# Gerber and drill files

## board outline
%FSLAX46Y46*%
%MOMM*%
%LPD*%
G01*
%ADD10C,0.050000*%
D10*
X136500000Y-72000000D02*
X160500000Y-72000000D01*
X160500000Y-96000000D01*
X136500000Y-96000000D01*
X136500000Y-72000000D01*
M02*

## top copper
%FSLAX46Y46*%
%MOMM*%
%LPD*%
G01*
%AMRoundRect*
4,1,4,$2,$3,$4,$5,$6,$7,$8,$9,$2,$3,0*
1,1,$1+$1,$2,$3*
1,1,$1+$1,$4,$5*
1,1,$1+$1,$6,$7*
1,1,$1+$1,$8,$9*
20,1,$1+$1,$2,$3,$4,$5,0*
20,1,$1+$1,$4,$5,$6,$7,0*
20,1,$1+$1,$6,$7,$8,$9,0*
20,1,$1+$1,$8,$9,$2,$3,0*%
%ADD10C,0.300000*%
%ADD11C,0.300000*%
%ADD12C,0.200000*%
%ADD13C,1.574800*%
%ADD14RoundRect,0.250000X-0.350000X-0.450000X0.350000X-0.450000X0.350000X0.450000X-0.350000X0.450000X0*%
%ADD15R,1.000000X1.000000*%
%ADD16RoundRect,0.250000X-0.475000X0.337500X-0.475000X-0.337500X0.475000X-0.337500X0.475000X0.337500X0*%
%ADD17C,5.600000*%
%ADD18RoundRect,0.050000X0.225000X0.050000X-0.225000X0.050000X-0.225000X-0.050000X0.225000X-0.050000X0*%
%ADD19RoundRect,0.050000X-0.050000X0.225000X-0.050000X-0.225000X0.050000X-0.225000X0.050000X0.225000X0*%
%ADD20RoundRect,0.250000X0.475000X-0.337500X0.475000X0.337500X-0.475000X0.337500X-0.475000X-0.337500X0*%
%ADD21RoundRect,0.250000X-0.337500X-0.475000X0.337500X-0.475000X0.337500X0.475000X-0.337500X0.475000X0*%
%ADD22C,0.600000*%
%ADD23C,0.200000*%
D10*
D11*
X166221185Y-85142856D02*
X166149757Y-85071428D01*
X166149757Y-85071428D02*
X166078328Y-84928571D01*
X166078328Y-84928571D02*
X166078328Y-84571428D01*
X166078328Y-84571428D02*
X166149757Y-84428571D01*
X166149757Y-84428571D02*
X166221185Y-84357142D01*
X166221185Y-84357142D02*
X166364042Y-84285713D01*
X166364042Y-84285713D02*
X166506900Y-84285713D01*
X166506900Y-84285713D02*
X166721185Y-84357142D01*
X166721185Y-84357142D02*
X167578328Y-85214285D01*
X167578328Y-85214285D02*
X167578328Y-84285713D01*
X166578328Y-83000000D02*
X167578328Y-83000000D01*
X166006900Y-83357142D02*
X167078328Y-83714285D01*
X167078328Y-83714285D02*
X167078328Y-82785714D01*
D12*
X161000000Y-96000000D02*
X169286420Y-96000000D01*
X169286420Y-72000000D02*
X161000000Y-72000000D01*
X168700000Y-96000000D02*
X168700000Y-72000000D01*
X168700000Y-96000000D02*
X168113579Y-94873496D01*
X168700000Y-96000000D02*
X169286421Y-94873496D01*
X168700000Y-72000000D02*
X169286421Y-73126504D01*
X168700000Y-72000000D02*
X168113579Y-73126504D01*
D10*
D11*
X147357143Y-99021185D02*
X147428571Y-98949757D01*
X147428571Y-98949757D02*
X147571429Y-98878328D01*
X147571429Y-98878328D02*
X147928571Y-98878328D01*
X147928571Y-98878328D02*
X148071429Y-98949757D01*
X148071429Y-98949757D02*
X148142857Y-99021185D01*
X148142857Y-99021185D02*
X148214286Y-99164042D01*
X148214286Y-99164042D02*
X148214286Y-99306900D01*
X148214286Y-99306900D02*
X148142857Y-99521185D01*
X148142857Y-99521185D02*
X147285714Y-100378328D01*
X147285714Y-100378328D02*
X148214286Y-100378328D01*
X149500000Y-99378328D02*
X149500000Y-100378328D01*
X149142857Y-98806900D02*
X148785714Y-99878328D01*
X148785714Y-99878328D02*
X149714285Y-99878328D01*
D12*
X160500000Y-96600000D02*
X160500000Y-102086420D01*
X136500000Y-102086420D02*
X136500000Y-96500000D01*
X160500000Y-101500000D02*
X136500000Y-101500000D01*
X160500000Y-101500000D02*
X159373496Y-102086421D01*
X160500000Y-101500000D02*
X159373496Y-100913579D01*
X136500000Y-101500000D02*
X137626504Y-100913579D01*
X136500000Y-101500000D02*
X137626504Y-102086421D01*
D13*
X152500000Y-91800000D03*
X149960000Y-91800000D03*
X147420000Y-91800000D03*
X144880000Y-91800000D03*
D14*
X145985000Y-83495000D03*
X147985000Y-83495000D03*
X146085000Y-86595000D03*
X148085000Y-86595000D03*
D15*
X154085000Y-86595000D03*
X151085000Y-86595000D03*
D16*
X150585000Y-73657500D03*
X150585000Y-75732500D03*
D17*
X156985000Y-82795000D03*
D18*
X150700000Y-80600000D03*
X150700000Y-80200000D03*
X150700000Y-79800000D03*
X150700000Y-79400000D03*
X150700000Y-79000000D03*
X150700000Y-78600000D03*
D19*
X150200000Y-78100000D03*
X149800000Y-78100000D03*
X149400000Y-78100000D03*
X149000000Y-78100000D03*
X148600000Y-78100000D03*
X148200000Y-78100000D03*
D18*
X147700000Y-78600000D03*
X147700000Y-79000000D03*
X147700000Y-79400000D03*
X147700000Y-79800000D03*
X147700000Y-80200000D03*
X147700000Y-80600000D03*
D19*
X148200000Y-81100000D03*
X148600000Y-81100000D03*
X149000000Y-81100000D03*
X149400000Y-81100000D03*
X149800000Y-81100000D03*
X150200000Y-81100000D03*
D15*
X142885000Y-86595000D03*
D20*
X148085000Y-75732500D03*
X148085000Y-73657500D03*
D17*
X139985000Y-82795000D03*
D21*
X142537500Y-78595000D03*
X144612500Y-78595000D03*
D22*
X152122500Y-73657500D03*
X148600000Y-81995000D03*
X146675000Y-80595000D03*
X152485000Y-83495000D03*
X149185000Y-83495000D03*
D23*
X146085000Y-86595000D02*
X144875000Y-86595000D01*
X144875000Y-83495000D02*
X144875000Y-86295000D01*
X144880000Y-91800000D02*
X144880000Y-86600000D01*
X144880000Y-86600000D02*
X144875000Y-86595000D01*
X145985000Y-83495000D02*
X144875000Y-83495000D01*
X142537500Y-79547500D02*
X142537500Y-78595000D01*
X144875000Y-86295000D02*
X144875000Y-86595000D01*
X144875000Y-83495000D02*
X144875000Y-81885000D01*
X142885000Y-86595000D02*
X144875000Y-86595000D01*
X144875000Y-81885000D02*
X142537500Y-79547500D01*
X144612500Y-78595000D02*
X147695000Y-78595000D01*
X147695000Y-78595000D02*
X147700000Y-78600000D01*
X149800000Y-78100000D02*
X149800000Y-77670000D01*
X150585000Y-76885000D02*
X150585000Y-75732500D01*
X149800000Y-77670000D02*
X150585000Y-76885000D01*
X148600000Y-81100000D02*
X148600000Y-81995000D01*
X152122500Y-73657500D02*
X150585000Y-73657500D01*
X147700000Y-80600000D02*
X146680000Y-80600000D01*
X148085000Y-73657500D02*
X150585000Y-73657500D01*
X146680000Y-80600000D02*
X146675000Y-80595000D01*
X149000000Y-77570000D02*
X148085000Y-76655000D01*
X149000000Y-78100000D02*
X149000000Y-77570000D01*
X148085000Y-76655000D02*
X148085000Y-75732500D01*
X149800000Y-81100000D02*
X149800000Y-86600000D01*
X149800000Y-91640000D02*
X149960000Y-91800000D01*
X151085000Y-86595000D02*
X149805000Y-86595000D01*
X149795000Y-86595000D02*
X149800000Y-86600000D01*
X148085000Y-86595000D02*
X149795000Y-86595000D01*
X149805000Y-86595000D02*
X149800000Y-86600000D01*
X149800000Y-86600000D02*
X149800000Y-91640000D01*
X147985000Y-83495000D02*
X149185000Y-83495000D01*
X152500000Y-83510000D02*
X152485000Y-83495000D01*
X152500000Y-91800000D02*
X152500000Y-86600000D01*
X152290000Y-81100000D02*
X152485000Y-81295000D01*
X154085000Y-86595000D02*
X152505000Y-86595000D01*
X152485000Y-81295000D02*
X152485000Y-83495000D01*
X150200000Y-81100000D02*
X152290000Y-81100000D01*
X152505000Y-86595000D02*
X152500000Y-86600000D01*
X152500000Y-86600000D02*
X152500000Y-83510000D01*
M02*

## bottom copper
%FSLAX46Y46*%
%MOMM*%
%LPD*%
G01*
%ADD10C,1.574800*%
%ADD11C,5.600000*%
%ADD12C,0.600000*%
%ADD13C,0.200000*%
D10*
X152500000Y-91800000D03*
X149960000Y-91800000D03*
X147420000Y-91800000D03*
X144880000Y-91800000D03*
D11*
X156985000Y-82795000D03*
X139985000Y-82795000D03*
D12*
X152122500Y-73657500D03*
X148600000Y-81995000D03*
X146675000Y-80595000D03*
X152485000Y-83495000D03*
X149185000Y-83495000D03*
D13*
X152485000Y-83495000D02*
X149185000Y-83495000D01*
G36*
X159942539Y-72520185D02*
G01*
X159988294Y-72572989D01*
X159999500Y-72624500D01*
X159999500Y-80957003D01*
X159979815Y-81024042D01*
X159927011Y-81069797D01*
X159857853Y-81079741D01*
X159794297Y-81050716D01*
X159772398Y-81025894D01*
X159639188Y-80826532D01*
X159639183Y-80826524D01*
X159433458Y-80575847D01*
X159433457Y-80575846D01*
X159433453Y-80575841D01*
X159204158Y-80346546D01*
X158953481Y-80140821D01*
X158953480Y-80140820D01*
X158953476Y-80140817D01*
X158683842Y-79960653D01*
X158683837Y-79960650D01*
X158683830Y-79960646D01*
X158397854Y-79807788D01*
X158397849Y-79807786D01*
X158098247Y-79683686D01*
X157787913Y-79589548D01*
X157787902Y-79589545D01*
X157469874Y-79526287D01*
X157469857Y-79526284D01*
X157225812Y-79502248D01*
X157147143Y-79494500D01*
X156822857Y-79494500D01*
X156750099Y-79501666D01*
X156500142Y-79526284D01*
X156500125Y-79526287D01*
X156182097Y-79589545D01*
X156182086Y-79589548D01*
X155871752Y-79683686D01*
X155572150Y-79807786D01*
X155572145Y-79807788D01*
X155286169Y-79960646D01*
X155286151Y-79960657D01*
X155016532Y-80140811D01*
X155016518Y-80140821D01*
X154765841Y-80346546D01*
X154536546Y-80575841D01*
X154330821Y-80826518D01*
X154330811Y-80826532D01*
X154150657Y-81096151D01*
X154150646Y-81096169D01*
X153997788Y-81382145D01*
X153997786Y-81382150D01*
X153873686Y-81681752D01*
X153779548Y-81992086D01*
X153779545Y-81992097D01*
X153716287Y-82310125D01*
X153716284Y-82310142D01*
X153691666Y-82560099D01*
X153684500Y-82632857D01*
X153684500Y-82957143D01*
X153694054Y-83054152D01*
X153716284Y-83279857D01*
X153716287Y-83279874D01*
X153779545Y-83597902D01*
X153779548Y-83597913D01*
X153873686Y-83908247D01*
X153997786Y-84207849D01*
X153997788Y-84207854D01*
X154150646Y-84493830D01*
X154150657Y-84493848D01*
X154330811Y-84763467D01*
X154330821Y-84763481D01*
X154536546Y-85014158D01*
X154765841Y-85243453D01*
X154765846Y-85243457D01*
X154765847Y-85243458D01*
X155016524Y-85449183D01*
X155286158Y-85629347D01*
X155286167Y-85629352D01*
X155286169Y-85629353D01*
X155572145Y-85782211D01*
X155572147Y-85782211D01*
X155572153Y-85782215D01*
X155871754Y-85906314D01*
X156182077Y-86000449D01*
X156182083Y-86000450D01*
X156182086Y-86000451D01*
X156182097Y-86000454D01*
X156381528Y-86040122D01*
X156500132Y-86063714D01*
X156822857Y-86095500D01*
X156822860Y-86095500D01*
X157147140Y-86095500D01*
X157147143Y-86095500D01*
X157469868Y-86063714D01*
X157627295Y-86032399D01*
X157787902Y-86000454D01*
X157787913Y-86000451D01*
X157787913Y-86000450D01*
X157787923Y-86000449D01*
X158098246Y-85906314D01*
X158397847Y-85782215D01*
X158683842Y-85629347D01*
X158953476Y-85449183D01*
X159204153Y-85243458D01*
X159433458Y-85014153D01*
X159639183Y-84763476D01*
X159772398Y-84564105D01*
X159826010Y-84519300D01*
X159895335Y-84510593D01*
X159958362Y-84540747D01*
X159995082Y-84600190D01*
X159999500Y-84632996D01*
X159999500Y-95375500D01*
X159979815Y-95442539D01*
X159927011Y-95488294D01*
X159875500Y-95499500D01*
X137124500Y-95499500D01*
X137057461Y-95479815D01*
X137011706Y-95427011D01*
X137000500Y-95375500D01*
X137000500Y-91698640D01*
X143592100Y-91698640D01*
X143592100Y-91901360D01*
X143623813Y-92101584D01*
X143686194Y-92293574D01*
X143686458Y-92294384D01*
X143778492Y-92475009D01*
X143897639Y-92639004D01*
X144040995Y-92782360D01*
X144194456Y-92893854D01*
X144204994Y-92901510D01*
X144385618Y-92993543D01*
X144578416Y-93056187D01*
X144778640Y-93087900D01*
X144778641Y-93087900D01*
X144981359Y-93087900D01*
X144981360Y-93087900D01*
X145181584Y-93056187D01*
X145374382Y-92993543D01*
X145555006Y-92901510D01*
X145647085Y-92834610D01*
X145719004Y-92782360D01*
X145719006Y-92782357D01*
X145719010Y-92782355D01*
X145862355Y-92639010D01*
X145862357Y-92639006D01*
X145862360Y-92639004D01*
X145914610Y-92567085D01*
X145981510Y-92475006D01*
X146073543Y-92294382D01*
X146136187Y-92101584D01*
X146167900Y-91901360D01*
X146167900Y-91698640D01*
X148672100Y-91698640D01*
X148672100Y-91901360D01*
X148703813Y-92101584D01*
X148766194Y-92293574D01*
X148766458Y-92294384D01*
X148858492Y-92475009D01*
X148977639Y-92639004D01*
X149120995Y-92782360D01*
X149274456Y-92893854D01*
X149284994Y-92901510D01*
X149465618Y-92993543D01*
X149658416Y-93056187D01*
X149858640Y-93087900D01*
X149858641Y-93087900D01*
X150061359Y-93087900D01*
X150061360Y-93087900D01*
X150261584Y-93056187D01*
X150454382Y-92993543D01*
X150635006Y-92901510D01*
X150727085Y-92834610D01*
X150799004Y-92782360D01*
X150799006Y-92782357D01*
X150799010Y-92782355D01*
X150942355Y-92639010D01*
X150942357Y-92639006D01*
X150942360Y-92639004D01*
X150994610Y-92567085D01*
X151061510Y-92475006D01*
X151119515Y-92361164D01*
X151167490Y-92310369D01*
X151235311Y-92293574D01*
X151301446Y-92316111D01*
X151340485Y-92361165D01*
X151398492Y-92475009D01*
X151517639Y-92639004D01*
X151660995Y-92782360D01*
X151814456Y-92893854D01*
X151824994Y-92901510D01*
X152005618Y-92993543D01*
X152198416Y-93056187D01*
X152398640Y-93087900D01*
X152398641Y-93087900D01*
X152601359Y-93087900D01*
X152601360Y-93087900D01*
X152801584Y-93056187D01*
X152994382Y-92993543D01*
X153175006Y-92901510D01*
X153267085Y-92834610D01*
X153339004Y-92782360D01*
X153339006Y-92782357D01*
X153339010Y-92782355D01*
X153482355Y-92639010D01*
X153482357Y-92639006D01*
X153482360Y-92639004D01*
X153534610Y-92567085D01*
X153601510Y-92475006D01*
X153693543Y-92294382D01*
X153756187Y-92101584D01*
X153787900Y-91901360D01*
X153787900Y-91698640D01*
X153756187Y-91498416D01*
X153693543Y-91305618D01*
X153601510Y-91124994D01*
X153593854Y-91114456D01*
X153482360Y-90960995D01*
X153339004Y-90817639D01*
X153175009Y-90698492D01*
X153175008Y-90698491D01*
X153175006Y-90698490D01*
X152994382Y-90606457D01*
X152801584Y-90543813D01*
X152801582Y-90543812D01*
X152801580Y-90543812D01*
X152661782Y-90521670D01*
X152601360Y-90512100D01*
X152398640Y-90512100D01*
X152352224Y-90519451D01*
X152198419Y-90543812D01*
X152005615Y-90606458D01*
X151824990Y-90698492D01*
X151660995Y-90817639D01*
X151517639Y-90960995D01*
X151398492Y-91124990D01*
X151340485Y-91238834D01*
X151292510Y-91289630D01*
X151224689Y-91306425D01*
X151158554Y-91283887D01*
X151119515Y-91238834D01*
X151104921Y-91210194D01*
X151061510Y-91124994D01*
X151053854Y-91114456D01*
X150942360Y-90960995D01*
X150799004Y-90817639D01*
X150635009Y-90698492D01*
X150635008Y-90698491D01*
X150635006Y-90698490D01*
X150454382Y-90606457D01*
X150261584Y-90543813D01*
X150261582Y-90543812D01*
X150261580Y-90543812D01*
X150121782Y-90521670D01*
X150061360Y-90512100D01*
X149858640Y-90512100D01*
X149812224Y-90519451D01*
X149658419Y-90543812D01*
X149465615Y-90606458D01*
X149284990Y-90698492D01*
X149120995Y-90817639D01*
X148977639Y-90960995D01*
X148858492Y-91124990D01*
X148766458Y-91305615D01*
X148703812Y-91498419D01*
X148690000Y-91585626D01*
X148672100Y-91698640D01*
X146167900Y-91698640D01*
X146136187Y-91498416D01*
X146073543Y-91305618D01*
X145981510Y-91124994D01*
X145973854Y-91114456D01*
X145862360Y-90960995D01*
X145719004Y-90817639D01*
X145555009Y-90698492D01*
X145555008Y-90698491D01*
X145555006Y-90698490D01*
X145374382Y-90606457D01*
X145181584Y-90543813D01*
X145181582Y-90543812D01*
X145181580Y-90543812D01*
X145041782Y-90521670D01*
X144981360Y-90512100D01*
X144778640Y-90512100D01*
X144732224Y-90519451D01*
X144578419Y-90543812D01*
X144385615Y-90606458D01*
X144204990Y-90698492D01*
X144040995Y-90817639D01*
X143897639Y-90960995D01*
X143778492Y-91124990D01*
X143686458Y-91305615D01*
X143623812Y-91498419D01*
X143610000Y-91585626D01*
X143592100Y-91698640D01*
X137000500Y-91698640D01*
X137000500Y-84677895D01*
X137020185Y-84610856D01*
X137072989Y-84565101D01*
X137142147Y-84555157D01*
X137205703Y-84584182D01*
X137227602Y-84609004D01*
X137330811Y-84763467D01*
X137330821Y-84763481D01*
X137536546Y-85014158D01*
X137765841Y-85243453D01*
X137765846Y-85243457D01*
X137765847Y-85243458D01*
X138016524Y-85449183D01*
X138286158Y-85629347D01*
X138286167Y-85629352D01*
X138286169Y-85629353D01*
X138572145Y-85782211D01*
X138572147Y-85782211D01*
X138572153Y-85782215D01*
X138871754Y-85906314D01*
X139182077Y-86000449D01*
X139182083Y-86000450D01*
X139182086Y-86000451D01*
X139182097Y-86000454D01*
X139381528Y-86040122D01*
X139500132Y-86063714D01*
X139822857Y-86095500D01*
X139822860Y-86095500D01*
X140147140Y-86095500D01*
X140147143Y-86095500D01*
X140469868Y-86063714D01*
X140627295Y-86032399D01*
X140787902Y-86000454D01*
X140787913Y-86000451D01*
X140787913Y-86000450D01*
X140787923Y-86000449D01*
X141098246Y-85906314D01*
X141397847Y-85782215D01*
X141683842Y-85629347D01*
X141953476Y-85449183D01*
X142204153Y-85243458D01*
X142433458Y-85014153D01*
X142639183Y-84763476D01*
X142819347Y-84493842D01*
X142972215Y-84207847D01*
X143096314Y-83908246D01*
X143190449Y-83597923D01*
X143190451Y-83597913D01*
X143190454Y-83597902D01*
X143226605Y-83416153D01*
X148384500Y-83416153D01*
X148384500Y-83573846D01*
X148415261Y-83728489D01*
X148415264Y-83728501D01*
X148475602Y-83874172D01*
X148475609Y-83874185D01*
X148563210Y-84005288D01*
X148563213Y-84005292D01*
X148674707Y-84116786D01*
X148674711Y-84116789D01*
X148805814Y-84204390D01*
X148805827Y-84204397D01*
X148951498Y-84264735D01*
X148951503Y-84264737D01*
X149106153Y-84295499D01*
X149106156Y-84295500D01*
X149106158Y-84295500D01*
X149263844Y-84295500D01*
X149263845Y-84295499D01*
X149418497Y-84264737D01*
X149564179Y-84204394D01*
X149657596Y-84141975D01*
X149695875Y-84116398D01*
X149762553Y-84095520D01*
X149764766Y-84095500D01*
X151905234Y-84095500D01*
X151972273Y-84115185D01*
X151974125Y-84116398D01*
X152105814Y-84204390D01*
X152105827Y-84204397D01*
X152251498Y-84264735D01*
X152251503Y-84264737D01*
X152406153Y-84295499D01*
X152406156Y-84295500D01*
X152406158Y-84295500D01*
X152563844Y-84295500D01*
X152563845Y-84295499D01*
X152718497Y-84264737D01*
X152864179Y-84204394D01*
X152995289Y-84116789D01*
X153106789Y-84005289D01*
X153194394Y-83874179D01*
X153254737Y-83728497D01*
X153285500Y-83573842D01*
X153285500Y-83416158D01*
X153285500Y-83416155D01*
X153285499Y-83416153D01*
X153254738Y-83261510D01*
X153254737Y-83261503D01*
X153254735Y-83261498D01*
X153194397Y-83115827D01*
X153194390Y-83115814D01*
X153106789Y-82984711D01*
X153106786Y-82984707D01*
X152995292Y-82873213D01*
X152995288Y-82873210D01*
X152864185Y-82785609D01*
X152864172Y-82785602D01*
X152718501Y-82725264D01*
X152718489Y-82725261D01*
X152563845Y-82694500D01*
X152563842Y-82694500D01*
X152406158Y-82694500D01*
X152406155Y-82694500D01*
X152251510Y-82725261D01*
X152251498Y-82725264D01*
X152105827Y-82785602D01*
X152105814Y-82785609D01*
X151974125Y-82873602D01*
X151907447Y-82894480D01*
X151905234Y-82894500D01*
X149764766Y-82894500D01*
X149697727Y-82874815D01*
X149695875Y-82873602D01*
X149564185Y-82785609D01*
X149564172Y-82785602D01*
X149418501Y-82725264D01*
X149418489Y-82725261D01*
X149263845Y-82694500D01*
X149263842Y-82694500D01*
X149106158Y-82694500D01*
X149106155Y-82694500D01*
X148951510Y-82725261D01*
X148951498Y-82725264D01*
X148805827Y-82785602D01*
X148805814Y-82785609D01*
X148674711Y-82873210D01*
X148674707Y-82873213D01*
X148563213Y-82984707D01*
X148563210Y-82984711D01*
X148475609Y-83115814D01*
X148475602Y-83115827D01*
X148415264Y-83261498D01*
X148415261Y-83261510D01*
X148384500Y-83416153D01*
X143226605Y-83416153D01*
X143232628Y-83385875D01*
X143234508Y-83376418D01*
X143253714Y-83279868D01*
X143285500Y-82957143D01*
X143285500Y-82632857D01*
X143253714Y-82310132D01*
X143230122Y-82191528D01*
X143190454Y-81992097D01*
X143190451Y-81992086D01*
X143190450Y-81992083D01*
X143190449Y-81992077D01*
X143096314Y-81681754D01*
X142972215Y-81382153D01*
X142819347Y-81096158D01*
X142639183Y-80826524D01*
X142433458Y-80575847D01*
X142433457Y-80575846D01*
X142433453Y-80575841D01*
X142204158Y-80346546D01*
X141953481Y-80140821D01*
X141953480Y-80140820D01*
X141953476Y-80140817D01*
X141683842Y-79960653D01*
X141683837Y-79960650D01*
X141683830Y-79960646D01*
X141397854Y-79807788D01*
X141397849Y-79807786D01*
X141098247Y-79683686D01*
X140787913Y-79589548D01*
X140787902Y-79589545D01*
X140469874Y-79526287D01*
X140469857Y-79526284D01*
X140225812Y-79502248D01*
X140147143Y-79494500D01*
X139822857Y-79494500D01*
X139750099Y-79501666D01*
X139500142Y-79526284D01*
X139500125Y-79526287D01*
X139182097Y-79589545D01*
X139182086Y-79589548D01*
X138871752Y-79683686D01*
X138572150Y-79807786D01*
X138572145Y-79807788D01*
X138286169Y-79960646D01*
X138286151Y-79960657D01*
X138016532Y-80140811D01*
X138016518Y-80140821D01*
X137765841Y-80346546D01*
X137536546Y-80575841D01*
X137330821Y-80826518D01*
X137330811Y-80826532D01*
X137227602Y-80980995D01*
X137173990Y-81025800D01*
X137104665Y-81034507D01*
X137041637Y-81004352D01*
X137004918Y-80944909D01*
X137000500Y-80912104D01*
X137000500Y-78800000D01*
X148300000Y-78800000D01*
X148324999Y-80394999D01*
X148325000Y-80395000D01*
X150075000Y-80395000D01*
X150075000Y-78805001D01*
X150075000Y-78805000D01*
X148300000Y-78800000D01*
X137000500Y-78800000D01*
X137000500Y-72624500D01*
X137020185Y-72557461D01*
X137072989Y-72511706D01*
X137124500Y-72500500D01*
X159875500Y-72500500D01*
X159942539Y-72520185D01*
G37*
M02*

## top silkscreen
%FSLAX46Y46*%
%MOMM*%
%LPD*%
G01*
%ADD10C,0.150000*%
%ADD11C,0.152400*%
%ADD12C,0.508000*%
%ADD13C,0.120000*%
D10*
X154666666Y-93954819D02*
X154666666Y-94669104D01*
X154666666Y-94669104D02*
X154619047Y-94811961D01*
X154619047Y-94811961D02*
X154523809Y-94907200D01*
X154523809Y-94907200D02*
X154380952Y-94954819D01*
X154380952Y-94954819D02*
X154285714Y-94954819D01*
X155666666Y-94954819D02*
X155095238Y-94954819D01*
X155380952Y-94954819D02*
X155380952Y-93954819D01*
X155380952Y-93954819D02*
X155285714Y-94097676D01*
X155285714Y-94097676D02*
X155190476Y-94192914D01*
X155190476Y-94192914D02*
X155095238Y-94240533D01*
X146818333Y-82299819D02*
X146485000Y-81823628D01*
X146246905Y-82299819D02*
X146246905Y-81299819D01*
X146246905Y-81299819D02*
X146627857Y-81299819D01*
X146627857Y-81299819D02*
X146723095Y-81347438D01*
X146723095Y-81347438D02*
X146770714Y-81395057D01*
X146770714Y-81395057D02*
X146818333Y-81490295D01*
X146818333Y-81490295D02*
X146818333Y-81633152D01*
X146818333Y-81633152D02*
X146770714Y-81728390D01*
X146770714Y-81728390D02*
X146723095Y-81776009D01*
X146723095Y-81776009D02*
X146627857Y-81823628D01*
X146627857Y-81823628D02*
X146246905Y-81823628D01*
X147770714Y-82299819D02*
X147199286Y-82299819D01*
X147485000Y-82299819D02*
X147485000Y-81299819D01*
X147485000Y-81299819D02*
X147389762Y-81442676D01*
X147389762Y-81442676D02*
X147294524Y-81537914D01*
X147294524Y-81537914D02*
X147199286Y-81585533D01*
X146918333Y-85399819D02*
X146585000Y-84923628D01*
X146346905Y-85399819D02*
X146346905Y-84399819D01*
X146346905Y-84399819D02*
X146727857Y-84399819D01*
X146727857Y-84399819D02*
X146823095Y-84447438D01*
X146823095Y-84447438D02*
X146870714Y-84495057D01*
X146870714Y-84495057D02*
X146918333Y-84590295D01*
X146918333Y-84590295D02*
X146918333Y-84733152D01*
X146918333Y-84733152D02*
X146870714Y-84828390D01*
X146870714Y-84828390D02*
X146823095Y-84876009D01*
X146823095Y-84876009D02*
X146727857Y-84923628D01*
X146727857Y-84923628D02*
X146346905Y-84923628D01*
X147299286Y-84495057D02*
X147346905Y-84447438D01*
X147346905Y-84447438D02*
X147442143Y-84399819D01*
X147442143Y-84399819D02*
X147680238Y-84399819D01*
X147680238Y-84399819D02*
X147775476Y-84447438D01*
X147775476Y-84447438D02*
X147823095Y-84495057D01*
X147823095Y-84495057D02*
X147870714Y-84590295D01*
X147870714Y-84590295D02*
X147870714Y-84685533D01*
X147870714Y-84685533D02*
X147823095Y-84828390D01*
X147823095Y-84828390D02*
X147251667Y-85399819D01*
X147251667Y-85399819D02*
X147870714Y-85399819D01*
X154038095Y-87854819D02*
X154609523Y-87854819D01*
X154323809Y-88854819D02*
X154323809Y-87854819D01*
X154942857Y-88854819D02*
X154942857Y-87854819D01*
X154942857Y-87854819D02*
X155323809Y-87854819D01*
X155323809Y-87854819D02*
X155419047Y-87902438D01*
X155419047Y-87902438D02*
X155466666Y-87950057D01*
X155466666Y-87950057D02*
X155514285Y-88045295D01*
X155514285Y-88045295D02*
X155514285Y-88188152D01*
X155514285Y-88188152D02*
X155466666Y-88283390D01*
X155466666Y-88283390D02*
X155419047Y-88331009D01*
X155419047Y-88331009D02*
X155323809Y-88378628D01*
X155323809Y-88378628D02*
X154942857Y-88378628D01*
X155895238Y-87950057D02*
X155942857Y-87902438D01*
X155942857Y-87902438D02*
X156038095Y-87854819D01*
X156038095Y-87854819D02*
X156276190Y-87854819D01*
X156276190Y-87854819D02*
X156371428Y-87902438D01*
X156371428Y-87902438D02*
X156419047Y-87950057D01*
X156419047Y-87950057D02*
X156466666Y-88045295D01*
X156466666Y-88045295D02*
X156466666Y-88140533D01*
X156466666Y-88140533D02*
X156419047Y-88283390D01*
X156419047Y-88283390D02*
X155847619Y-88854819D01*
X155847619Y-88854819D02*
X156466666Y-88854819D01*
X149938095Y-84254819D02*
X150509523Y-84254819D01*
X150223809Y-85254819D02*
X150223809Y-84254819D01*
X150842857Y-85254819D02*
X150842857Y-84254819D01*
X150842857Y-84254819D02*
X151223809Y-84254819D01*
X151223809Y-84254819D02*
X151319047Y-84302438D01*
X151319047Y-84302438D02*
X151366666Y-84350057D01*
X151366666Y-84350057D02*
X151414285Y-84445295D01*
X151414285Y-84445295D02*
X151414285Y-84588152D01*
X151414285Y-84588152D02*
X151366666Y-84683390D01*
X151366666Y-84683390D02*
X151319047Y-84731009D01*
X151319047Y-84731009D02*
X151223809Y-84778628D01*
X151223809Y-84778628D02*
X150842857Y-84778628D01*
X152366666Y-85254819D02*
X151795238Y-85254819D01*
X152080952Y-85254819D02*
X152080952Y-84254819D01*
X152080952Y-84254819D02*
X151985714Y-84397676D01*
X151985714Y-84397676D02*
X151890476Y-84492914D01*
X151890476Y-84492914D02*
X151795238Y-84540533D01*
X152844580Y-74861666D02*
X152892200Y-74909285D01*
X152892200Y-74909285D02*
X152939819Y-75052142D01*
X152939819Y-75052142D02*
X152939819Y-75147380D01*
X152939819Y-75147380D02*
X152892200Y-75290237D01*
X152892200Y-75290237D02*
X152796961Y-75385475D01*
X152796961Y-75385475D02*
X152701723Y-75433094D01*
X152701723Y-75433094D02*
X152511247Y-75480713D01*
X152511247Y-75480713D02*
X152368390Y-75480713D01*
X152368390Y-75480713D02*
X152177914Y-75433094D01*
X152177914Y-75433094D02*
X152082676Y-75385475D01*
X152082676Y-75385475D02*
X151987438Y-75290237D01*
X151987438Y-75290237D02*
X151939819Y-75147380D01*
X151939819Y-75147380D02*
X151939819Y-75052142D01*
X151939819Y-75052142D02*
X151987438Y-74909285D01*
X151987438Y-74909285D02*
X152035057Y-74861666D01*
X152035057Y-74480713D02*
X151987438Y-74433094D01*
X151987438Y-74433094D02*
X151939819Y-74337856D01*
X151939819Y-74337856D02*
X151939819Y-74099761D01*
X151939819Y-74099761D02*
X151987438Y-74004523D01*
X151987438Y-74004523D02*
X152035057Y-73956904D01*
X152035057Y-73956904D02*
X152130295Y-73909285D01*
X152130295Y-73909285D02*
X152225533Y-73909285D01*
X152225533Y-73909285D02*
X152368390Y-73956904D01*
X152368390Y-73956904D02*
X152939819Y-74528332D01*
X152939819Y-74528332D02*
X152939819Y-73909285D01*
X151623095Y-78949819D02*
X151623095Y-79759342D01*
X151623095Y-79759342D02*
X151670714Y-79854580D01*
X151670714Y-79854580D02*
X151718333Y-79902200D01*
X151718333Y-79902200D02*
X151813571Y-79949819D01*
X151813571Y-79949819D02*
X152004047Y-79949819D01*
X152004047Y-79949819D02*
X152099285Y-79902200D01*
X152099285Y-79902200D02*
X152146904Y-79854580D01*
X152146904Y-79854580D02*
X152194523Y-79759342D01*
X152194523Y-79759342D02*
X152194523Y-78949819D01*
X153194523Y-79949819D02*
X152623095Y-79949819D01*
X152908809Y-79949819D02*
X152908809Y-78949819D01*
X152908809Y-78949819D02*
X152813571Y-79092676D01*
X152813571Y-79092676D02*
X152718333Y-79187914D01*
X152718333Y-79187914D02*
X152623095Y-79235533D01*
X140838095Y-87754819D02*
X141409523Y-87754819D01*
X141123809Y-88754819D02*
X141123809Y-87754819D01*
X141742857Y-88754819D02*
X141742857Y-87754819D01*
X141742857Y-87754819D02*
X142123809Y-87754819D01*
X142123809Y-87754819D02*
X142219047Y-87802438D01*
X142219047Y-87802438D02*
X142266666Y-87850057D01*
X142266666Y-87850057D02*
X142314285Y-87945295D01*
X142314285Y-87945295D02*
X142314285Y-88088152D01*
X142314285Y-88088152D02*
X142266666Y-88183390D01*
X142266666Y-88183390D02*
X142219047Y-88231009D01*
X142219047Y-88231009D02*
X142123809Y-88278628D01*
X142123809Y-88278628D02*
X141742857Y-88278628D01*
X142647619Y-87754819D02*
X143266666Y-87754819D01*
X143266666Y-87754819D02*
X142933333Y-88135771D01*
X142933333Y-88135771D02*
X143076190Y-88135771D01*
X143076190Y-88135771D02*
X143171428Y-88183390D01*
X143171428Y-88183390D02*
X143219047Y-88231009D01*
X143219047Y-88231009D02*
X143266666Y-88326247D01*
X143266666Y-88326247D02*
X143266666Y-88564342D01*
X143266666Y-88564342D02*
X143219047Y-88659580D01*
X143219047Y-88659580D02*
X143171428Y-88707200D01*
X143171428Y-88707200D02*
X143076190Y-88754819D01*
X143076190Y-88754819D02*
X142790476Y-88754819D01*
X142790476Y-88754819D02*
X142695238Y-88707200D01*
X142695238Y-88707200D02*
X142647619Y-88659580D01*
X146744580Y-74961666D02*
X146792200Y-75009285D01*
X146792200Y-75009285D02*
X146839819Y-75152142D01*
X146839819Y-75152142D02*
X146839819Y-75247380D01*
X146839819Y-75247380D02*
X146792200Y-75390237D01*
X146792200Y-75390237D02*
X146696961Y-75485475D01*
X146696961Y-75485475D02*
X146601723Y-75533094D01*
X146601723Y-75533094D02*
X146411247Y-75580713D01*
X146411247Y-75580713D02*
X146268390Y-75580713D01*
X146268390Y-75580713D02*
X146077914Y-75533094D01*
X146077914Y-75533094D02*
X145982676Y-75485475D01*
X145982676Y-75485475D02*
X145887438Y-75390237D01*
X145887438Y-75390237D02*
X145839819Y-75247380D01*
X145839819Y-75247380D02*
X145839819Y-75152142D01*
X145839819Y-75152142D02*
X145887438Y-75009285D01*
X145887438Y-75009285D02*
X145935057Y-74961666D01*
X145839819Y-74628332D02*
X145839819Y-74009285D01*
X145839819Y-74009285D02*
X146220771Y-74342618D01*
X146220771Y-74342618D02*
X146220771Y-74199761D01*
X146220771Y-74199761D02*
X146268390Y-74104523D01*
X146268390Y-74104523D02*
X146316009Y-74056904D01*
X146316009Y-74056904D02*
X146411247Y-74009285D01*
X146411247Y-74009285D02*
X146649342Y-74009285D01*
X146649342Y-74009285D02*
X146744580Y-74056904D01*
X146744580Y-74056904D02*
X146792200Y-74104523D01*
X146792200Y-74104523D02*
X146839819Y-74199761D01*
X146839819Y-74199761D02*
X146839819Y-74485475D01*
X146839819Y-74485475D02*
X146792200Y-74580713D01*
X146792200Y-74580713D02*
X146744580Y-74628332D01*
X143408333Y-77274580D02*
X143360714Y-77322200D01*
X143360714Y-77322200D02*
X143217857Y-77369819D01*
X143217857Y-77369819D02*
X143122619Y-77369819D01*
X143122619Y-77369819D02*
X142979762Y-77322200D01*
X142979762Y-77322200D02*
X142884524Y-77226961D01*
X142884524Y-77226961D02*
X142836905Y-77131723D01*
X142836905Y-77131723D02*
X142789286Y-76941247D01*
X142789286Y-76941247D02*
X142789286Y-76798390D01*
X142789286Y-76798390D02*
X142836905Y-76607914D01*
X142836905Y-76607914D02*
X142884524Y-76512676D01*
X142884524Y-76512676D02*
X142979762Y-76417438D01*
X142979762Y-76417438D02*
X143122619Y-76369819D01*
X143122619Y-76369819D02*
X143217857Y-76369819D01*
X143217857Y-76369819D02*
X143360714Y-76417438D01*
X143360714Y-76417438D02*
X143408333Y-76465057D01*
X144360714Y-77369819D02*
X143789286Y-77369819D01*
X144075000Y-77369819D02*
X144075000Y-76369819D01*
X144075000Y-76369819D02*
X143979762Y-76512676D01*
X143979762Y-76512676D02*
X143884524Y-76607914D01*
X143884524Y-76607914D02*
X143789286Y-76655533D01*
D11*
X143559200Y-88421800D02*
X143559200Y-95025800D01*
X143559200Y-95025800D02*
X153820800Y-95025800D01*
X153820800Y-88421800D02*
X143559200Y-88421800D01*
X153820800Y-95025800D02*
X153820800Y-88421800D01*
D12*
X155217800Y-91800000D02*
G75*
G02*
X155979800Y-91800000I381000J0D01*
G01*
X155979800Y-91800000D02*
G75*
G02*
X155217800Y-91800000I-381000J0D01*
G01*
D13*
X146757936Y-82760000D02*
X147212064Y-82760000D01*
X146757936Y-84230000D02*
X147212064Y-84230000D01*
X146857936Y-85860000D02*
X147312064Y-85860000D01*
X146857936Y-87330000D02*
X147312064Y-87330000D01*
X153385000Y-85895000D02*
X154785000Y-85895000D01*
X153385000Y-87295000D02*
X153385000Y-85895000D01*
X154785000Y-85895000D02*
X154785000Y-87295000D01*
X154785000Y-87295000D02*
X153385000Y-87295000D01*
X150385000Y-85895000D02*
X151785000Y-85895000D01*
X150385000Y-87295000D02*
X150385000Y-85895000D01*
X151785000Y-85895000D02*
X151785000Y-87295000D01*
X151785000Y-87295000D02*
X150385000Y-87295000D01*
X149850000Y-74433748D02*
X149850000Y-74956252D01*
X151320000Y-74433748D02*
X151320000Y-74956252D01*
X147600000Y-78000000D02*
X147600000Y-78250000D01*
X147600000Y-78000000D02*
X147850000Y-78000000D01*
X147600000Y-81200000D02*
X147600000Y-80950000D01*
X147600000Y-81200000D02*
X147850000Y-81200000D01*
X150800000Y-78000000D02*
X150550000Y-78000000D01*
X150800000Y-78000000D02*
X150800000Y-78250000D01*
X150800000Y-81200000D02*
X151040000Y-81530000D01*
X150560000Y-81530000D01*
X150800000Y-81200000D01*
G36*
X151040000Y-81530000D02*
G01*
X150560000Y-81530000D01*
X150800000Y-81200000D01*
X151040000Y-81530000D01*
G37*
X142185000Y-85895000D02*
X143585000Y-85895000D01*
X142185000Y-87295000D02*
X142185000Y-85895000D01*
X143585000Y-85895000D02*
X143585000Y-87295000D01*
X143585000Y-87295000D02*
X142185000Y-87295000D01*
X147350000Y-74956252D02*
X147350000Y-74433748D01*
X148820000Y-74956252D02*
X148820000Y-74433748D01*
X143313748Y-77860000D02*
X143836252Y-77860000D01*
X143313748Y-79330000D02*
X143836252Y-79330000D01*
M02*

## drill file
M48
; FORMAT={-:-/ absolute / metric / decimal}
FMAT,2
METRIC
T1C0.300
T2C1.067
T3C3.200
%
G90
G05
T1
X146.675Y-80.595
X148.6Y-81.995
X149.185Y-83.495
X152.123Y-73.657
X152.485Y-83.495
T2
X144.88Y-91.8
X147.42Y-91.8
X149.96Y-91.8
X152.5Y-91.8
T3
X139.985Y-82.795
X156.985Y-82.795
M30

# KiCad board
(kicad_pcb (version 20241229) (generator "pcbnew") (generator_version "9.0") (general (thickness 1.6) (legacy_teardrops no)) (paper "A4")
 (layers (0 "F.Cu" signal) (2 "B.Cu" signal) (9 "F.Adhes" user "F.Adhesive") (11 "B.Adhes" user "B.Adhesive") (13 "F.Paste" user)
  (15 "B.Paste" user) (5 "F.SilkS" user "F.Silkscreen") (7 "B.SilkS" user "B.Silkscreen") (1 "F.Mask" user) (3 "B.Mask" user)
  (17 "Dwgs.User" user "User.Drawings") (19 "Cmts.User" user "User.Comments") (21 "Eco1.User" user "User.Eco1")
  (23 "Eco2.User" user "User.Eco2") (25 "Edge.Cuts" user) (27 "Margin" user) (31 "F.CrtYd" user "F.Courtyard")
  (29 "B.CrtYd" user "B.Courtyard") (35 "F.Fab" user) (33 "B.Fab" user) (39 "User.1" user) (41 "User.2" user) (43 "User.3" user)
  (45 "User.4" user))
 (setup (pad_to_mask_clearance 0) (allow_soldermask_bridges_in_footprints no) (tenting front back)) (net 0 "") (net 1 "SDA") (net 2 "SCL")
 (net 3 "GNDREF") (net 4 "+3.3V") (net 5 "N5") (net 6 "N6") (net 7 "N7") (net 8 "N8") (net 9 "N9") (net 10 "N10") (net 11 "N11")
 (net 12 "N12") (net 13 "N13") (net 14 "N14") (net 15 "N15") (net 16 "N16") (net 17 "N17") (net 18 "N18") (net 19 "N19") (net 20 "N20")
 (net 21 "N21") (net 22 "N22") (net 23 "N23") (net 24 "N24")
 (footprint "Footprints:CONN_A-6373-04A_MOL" (layer "F.Cu") (at 152.5 91.8 180)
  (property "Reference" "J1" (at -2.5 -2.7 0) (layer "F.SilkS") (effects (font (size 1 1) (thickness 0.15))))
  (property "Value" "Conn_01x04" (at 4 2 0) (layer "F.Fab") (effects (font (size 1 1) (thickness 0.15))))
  (fp_line (start 8.9408 3.3782) (end 8.9408 -3.2258) (stroke (width 0.1524) (type solid)) (layer "F.SilkS"))
  (fp_line (start 8.9408 -3.2258) (end -1.3208 -3.2258) (stroke (width 0.1524) (type solid)) (layer "F.SilkS"))
  (fp_line (start -1.3208 3.3782) (end 8.9408 3.3782) (stroke (width 0.1524) (type solid)) (layer "F.SilkS"))
  (fp_line (start -1.3208 -3.2258) (end -1.3208 3.3782) (stroke (width 0.1524) (type solid)) (layer "F.SilkS"))
  (fp_arc (start -2.7178 0) (mid -3.0988 0.381) (end -3.4798 0) (stroke (width 0.508) (type solid)) (layer "F.SilkS"))
  (fp_arc (start -3.4798 0) (mid -3.0988 -0.381) (end -2.7178 0) (stroke (width 0.508) (type solid)) (layer "F.SilkS"))
  (pad "1" thru_hole circle (at 0 0 180) (size 1.5748 1.5748) (drill 1.0668) (layers "*.Cu" "*.Mask") (remove_unused_layers no)
   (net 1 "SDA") (solder_mask_margin 0.102))
  (pad "2" thru_hole circle (at 2.54 0 180) (size 1.5748 1.5748) (drill 1.0668) (layers "*.Cu" "*.Mask") (remove_unused_layers no)
   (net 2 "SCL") (solder_mask_margin 0.102))
  (pad "3" thru_hole circle (at 5.08 0 180) (size 1.5748 1.5748) (drill 1.0668) (layers "*.Cu" "*.Mask") (remove_unused_layers no)
   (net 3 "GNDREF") (solder_mask_margin 0.102))
  (pad "4" thru_hole circle (at 7.62 0 180) (size 1.5748 1.5748) (drill 1.0668) (layers "*.Cu" "*.Mask") (remove_unused_layers no)
   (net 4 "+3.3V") (solder_mask_margin 0.102)))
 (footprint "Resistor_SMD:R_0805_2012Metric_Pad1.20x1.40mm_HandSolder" (layer "F.Cu") (at 146.985 83.495)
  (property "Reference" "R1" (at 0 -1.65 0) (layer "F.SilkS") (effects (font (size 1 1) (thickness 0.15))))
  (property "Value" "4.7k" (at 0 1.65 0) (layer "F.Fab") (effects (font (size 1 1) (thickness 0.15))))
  (fp_line (start -0.227064 -0.735) (end 0.227064 -0.735) (stroke (width 0.12) (type solid)) (layer "F.SilkS"))
  (fp_line (start -0.227064 0.735) (end 0.227064 0.735) (stroke (width 0.12) (type solid)) (layer "F.SilkS"))
  (pad "1" smd roundrect (at -1 0) (size 1.2 1.4) (layers "F.Cu" "F.Mask" "F.Paste") (roundrect_rratio 0.208333) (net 4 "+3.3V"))
  (pad "2" smd roundrect (at 1 0) (size 1.2 1.4) (layers "F.Cu" "F.Mask" "F.Paste") (roundrect_rratio 0.208333) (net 1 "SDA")))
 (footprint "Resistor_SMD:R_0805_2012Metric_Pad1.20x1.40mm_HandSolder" (layer "F.Cu") (at 147.085 86.595)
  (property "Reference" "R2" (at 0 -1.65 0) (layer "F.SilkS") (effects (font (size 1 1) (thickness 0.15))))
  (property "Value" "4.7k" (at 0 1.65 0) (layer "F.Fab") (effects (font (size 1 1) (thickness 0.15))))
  (fp_line (start -0.227064 -0.735) (end 0.227064 -0.735) (stroke (width 0.12) (type solid)) (layer "F.SilkS"))
  (fp_line (start -0.227064 0.735) (end 0.227064 0.735) (stroke (width 0.12) (type solid)) (layer "F.SilkS"))
  (pad "1" smd roundrect (at -1 0) (size 1.2 1.4) (layers "F.Cu" "F.Mask" "F.Paste") (roundrect_rratio 0.208333) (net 4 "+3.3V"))
  (pad "2" smd roundrect (at 1 0) (size 1.2 1.4) (layers "F.Cu" "F.Mask" "F.Paste") (roundrect_rratio 0.208333) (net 2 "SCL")))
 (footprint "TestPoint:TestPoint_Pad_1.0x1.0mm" (layer "F.Cu") (at 154.085 86.595)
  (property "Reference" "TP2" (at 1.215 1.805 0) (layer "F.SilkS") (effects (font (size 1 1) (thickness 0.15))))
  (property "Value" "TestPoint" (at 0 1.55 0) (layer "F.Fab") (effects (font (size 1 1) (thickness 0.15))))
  (fp_line (start -0.7 -0.7) (end 0.7 -0.7) (stroke (width 0.12) (type solid)) (layer "F.SilkS"))
  (fp_line (start -0.7 0.7) (end -0.7 -0.7) (stroke (width 0.12) (type solid)) (layer "F.SilkS"))
  (fp_line (start 0.7 -0.7) (end 0.7 0.7) (stroke (width 0.12) (type solid)) (layer "F.SilkS"))
  (fp_line (start 0.7 0.7) (end -0.7 0.7) (stroke (width 0.12) (type solid)) (layer "F.SilkS"))
  (pad "1" smd rect (at 0 0) (size 1 1) (layers "F.Cu" "F.Mask") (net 1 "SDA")))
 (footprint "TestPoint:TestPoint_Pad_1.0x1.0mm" (layer "F.Cu") (at 151.085 86.595)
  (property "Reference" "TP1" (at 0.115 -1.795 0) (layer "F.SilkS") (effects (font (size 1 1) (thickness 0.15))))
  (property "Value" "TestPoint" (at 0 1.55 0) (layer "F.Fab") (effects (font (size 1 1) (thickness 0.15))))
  (fp_line (start -0.7 -0.7) (end 0.7 -0.7) (stroke (width 0.12) (type solid)) (layer "F.SilkS"))
  (fp_line (start -0.7 0.7) (end -0.7 -0.7) (stroke (width 0.12) (type solid)) (layer "F.SilkS"))
  (fp_line (start 0.7 -0.7) (end 0.7 0.7) (stroke (width 0.12) (type solid)) (layer "F.SilkS"))
  (fp_line (start 0.7 0.7) (end -0.7 0.7) (stroke (width 0.12) (type solid)) (layer "F.SilkS"))
  (pad "1" smd rect (at 0 0) (size 1 1) (layers "F.Cu" "F.Mask") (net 2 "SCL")))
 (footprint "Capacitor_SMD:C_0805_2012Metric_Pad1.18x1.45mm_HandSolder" (layer "F.Cu") (at 150.585 74.695 -90)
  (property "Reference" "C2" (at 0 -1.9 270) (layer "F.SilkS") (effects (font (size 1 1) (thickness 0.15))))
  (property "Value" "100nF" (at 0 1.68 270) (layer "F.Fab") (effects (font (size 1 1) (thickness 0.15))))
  (fp_line (start -0.261252 0.735) (end 0.261252 0.735) (stroke (width 0.12) (type solid)) (layer "F.SilkS"))
  (fp_line (start -0.261252 -0.735) (end 0.261252 -0.735) (stroke (width 0.12) (type solid)) (layer "F.SilkS"))
  (pad "1" smd roundrect (at -1.0375 0 270) (size 1.175 1.45) (layers "F.Cu" "F.Mask" "F.Paste") (roundrect_rratio 0.212766)
   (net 3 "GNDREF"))
  (pad "2" smd roundrect (at 1.0375 0 270) (size 1.175 1.45) (layers "F.Cu" "F.Mask" "F.Paste") (roundrect_rratio 0.212766) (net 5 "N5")))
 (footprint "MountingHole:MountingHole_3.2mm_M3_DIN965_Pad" (layer "F.Cu") (at 156.985 82.795)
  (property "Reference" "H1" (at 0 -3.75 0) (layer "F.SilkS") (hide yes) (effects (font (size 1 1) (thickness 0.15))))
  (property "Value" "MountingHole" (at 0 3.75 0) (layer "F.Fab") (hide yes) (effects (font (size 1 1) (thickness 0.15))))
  (pad "1" thru_hole circle (at 0 0) (size 5.6 5.6) (drill 3.2) (layers "*.Cu" "*.Mask") (remove_unused_layers no) (zone_connect 2)))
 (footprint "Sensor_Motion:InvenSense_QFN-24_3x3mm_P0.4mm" (layer "F.Cu") (at 149.2 79.6 180)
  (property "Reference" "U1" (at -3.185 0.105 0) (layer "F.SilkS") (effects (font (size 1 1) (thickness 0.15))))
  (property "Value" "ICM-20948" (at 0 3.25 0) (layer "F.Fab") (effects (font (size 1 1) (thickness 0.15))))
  (fp_line (start 1.6 1.6) (end 1.6 1.35) (stroke (width 0.12) (type solid)) (layer "F.SilkS"))
  (fp_line (start 1.6 1.6) (end 1.35 1.6) (stroke (width 0.12) (type solid)) (layer "F.SilkS"))
  (fp_line (start 1.6 -1.6) (end 1.6 -1.35) (stroke (width 0.12) (type solid)) (layer "F.SilkS"))
  (fp_line (start 1.6 -1.6) (end 1.35 -1.6) (stroke (width 0.12) (type solid)) (layer "F.SilkS"))
  (fp_line (start -1.6 1.6) (end -1.35 1.6) (stroke (width 0.12) (type solid)) (layer "F.SilkS"))
  (fp_line (start -1.6 1.6) (end -1.6 1.35) (stroke (width 0.12) (type solid)) (layer "F.SilkS"))
  (fp_poly
   (pts (xy -1.6 -1.6) (xy -1.84 -1.93) (xy -1.36 -1.93) (xy -1.6 -1.6)) (stroke (width 0.12) (type solid)) (fill yes) (layer "F.SilkS"))
  (pad "1" smd roundrect (at -1.5 -1 180) (size 0.55 0.2) (layers "F.Cu" "F.Mask" "F.Paste") (roundrect_rratio 0.25) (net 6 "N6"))
  (pad "2" smd roundrect (at -1.5 -0.6 180) (size 0.55 0.2) (layers "F.Cu" "F.Mask" "F.Paste") (roundrect_rratio 0.25) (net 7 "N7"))
  (pad "3" smd roundrect (at -1.5 -0.2 180) (size 0.55 0.2) (layers "F.Cu" "F.Mask" "F.Paste") (roundrect_rratio 0.25) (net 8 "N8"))
  (pad "4" smd roundrect (at -1.5 0.2 180) (size 0.55 0.2) (layers "F.Cu" "F.Mask" "F.Paste") (roundrect_rratio 0.25) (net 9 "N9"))
  (pad "5" smd roundrect (at -1.5 0.6 180) (size 0.55 0.2) (layers "F.Cu" "F.Mask" "F.Paste") (roundrect_rratio 0.25) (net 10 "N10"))
  (pad "6" smd roundrect (at -1.5 1 180) (size 0.55 0.2) (layers "F.Cu" "F.Mask" "F.Paste") (roundrect_rratio 0.25) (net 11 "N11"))
  (pad "7" smd roundrect (at -1 1.5 270) (size 0.55 0.2) (layers "F.Cu" "F.Mask" "F.Paste") (roundrect_rratio 0.25) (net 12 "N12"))
  (pad "8" smd roundrect (at -0.6 1.5 270) (size 0.55 0.2) (layers "F.Cu" "F.Mask" "F.Paste") (roundrect_rratio 0.25) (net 5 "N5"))
  (pad "9" smd roundrect (at -0.2 1.5 270) (size 0.55 0.2) (layers "F.Cu" "F.Mask" "F.Paste") (roundrect_rratio 0.25) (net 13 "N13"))
  (pad "10" smd roundrect (at 0.2 1.5 270) (size 0.55 0.2) (layers "F.Cu" "F.Mask" "F.Paste") (roundrect_rratio 0.25) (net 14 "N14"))
  (pad "11" smd roundrect (at 0.6 1.5 270) (size 0.55 0.2) (layers "F.Cu" "F.Mask" "F.Paste") (roundrect_rratio 0.25) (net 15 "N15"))
  (pad "12" smd roundrect (at 1 1.5 270) (size 0.55 0.2) (layers "F.Cu" "F.Mask" "F.Paste") (roundrect_rratio 0.25) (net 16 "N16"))
  (pad "13" smd roundrect (at 1.5 1 180) (size 0.55 0.2) (layers "F.Cu" "F.Mask" "F.Paste") (roundrect_rratio 0.25) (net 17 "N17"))
  (pad "14" smd roundrect (at 1.5 0.6 180) (size 0.55 0.2) (layers "F.Cu" "F.Mask" "F.Paste") (roundrect_rratio 0.25) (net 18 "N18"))
  (pad "15" smd roundrect (at 1.5 0.2 180) (size 0.55 0.2) (layers "F.Cu" "F.Mask" "F.Paste") (roundrect_rratio 0.25) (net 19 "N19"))
  (pad "16" smd roundrect (at 1.5 -0.2 180) (size 0.55 0.2) (layers "F.Cu" "F.Mask" "F.Paste") (roundrect_rratio 0.25) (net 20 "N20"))
  (pad "17" smd roundrect (at 1.5 -0.6 180) (size 0.55 0.2) (layers "F.Cu" "F.Mask" "F.Paste") (roundrect_rratio 0.25) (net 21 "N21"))
  (pad "18" smd roundrect (at 1.5 -1 180) (size 0.55 0.2) (layers "F.Cu" "F.Mask" "F.Paste") (roundrect_rratio 0.25) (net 3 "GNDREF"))
  (pad "19" smd roundrect (at 1 -1.5 270) (size 0.55 0.2) (layers "F.Cu" "F.Mask" "F.Paste") (roundrect_rratio 0.25) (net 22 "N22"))
  (pad "20" smd roundrect (at 0.6 -1.5 270) (size 0.55 0.2) (layers "F.Cu" "F.Mask" "F.Paste") (roundrect_rratio 0.25) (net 3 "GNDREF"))
  (pad "21" smd roundrect (at 0.2 -1.5 270) (size 0.55 0.2) (layers "F.Cu" "F.Mask" "F.Paste") (roundrect_rratio 0.25) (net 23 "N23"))
  (pad "22" smd roundrect (at -0.2 -1.5 270) (size 0.55 0.2) (layers "F.Cu" "F.Mask" "F.Paste") (roundrect_rratio 0.25) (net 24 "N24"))
  (pad "23" smd roundrect (at -0.6 -1.5 270) (size 0.55 0.2) (layers "F.Cu" "F.Mask" "F.Paste") (roundrect_rratio 0.25) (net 2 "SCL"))
  (pad "24" smd roundrect (at -1 -1.5 270) (size 0.55 0.2) (layers "F.Cu" "F.Mask" "F.Paste") (roundrect_rratio 0.25) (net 1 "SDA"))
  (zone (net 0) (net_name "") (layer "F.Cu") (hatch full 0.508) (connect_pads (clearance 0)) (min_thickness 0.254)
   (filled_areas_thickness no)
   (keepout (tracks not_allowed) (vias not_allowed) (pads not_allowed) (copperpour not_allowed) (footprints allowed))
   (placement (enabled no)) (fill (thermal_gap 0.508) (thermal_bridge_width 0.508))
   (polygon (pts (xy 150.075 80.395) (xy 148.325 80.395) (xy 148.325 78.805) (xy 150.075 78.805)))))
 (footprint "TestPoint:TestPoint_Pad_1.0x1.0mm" (layer "F.Cu") (at 142.885 86.595)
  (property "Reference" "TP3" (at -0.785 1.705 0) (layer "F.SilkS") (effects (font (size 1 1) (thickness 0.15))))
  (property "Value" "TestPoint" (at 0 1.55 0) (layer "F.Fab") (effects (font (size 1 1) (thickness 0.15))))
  (fp_line (start -0.7 -0.7) (end 0.7 -0.7) (stroke (width 0.12) (type solid)) (layer "F.SilkS"))
  (fp_line (start -0.7 0.7) (end -0.7 -0.7) (stroke (width 0.12) (type solid)) (layer "F.SilkS"))
  (fp_line (start 0.7 -0.7) (end 0.7 0.7) (stroke (width 0.12) (type solid)) (layer "F.SilkS"))
  (fp_line (start 0.7 0.7) (end -0.7 0.7) (stroke (width 0.12) (type solid)) (layer "F.SilkS"))
  (pad "1" smd rect (at 0 0) (size 1 1) (layers "F.Cu" "F.Mask") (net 4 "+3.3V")))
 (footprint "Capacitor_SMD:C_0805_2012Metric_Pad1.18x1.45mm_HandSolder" (layer "F.Cu") (at 148.085 74.695 90)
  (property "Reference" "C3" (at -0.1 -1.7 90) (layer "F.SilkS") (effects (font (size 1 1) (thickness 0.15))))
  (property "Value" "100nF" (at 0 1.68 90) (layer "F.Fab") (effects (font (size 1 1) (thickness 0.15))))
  (fp_line (start -0.261252 -0.735) (end 0.261252 -0.735) (stroke (width 0.12) (type solid)) (layer "F.SilkS"))
  (fp_line (start -0.261252 0.735) (end 0.261252 0.735) (stroke (width 0.12) (type solid)) (layer "F.SilkS"))
  (pad "1" smd roundrect (at -1.0375 0 90) (size 1.175 1.45) (layers "F.Cu" "F.Mask" "F.Paste") (roundrect_rratio 0.212766) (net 14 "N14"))
  (pad "2" smd roundrect (at 1.0375 0 90) (size 1.175 1.45) (layers "F.Cu" "F.Mask" "F.Paste") (roundrect_rratio 0.212766) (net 3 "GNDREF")))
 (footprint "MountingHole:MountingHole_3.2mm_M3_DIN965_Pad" (layer "F.Cu") (at 139.985 82.795)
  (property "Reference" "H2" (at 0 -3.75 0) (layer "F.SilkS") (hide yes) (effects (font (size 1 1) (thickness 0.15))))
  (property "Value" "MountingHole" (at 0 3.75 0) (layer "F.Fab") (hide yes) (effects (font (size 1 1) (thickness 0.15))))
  (pad "1" thru_hole circle (at 0 0) (size 5.6 5.6) (drill 3.2) (layers "*.Cu" "*.Mask") (remove_unused_layers no) (zone_connect 2)))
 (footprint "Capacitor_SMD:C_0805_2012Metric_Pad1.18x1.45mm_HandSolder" (layer "F.Cu") (at 143.575 78.595)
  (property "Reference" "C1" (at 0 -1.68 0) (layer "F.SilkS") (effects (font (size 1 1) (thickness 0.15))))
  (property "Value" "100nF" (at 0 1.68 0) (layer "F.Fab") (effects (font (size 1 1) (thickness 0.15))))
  (fp_line (start -0.261252 -0.735) (end 0.261252 -0.735) (stroke (width 0.12) (type solid)) (layer "F.SilkS"))
  (fp_line (start -0.261252 0.735) (end 0.261252 0.735) (stroke (width 0.12) (type solid)) (layer "F.SilkS"))
  (pad "1" smd roundrect (at -1.0375 0) (size 1.175 1.45) (layers "F.Cu" "F.Mask" "F.Paste") (roundrect_rratio 0.212766) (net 4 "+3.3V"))
  (pad "2" smd roundrect (at 1.0375 0) (size 1.175 1.45) (layers "F.Cu" "F.Mask" "F.Paste") (roundrect_rratio 0.212766) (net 17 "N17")))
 (gr_rect (start 136.5 72) (end 160.5 96) (stroke (width 0.05) (type default)) (fill no) (layer "Edge.Cuts"))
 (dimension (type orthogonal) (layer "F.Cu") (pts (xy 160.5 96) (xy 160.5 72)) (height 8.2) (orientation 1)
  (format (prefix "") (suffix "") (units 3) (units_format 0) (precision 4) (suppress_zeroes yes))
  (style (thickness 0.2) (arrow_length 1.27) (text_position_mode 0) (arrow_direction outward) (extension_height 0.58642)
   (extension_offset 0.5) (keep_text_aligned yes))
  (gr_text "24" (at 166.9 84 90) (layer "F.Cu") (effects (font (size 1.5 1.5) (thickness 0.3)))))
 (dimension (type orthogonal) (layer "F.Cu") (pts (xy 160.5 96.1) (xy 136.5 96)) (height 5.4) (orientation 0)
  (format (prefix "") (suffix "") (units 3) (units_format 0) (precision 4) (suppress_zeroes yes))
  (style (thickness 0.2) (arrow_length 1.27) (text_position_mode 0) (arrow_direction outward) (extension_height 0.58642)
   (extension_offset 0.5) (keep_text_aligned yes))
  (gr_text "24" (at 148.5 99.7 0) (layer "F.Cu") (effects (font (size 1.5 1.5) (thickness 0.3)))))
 (segment (start 146.085 86.595) (end 144.875 86.595) (width 0.2) (layer "F.Cu") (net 4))
 (segment (start 144.875 83.495) (end 144.875 86.295) (width 0.2) (layer "F.Cu") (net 4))
 (segment (start 144.88 91.8) (end 144.88 86.6) (width 0.2) (layer "F.Cu") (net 4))
 (segment (start 144.88 86.6) (end 144.875 86.595) (width 0.2) (layer "F.Cu") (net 4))
 (segment (start 145.985 83.495) (end 144.875 83.495) (width 0.2) (layer "F.Cu") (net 4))
 (segment (start 142.5375 79.5475) (end 142.5375 78.595) (width 0.2) (layer "F.Cu") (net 4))
 (segment (start 144.875 86.295) (end 144.875 86.595) (width 0.2) (layer "F.Cu") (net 4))
 (segment (start 144.875 83.495) (end 144.875 81.885) (width 0.2) (layer "F.Cu") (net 4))
 (segment (start 142.885 86.595) (end 144.875 86.595) (width 0.2) (layer "F.Cu") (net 4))
 (segment (start 144.875 81.885) (end 142.5375 79.5475) (width 0.2) (layer "F.Cu") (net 4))
 (segment (start 144.6125 78.595) (end 147.695 78.595) (width 0.2) (layer "F.Cu") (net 17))
 (segment (start 147.695 78.595) (end 147.7 78.6) (width 0.2) (layer "F.Cu") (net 17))
 (segment (start 149.8 78.1) (end 149.8 77.67) (width 0.2) (layer "F.Cu") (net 5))
 (segment (start 150.585 76.885) (end 150.585 75.7325) (width 0.2) (layer "F.Cu") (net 5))
 (segment (start 149.8 77.67) (end 150.585 76.885) (width 0.2) (layer "F.Cu") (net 5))
 (segment (start 148.6 81.1) (end 148.6 81.995) (width 0.2) (layer "F.Cu") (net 3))
 (segment (start 152.1225 73.6575) (end 150.585 73.6575) (width 0.2) (layer "F.Cu") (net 3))
 (segment (start 147.7 80.6) (end 146.68 80.6) (width 0.2) (layer "F.Cu") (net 3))
 (segment (start 148.085 73.6575) (end 150.585 73.6575) (width 0.2) (layer "F.Cu") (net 3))
 (segment (start 146.68 80.6) (end 146.675 80.595) (width 0.2) (layer "F.Cu") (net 3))
 (via (at 152.1225 73.6575) (size 0.6) (drill 0.3) (layers "F.Cu" "B.Cu") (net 3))
 (via (at 148.6 81.995) (size 0.6) (drill 0.3) (layers "F.Cu" "B.Cu") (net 3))
 (via (at 146.675 80.595) (size 0.6) (drill 0.3) (layers "F.Cu" "B.Cu") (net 3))
 (segment (start 149 77.57) (end 148.085 76.655) (width 0.2) (layer "F.Cu") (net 14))
 (segment (start 149 78.1) (end 149 77.57) (width 0.2) (layer "F.Cu") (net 14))
 (segment (start 148.085 76.655) (end 148.085 75.7325) (width 0.2) (layer "F.Cu") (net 14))
 (segment (start 149.8 81.1) (end 149.8 86.6) (width 0.2) (layer "F.Cu") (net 2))
 (segment (start 149.8 91.64) (end 149.96 91.8) (width 0.2) (layer "F.Cu") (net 2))
 (segment (start 151.085 86.595) (end 149.805 86.595) (width 0.2) (layer "F.Cu") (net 2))
 (segment (start 149.795 86.595) (end 149.8 86.6) (width 0.2) (layer "F.Cu") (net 2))
 (segment (start 148.085 86.595) (end 149.795 86.595) (width 0.2) (layer "F.Cu") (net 2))
 (segment (start 149.805 86.595) (end 149.8 86.6) (width 0.2) (layer "F.Cu") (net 2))
 (segment (start 149.8 86.6) (end 149.8 91.64) (width 0.2) (layer "F.Cu") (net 2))
 (segment (start 147.985 83.495) (end 149.185 83.495) (width 0.2) (layer "F.Cu") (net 1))
 (segment (start 152.5 83.51) (end 152.485 83.495) (width 0.2) (layer "F.Cu") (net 1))
 (segment (start 152.5 91.8) (end 152.5 86.6) (width 0.2) (layer "F.Cu") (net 1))
 (segment (start 152.29 81.1) (end 152.485 81.295) (width 0.2) (layer "F.Cu") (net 1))
 (segment (start 154.085 86.595) (end 152.505 86.595) (width 0.2) (layer "F.Cu") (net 1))
 (segment (start 152.485 81.295) (end 152.485 83.495) (width 0.2) (layer "F.Cu") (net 1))
 (segment (start 150.2 81.1) (end 152.29 81.1) (width 0.2) (layer "F.Cu") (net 1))
 (segment (start 152.505 86.595) (end 152.5 86.6) (width 0.2) (layer "F.Cu") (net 1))
 (segment (start 152.5 86.6) (end 152.5 83.51) (width 0.2) (layer "F.Cu") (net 1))
 (via (at 152.485 83.495) (size 0.6) (drill 0.3) (layers "F.Cu" "B.Cu") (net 1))
 (via (at 149.185 83.495) (size 0.6) (drill 0.3) (layers "F.Cu" "B.Cu") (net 1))
 (segment (start 152.485 83.495) (end 149.185 83.495) (width 0.2) (layer "B.Cu") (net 1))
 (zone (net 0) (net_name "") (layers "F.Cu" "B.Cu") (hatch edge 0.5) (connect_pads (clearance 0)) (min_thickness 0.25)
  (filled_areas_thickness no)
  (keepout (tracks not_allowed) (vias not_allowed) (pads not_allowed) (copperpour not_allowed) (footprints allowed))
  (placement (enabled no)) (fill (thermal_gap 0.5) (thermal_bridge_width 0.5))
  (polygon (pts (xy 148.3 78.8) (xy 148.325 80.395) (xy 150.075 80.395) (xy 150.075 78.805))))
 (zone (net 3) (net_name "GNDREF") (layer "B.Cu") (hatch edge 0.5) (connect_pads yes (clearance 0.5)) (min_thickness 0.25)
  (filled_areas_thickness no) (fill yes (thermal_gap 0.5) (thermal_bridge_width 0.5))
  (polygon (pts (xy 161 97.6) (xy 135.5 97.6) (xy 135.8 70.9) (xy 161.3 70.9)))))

